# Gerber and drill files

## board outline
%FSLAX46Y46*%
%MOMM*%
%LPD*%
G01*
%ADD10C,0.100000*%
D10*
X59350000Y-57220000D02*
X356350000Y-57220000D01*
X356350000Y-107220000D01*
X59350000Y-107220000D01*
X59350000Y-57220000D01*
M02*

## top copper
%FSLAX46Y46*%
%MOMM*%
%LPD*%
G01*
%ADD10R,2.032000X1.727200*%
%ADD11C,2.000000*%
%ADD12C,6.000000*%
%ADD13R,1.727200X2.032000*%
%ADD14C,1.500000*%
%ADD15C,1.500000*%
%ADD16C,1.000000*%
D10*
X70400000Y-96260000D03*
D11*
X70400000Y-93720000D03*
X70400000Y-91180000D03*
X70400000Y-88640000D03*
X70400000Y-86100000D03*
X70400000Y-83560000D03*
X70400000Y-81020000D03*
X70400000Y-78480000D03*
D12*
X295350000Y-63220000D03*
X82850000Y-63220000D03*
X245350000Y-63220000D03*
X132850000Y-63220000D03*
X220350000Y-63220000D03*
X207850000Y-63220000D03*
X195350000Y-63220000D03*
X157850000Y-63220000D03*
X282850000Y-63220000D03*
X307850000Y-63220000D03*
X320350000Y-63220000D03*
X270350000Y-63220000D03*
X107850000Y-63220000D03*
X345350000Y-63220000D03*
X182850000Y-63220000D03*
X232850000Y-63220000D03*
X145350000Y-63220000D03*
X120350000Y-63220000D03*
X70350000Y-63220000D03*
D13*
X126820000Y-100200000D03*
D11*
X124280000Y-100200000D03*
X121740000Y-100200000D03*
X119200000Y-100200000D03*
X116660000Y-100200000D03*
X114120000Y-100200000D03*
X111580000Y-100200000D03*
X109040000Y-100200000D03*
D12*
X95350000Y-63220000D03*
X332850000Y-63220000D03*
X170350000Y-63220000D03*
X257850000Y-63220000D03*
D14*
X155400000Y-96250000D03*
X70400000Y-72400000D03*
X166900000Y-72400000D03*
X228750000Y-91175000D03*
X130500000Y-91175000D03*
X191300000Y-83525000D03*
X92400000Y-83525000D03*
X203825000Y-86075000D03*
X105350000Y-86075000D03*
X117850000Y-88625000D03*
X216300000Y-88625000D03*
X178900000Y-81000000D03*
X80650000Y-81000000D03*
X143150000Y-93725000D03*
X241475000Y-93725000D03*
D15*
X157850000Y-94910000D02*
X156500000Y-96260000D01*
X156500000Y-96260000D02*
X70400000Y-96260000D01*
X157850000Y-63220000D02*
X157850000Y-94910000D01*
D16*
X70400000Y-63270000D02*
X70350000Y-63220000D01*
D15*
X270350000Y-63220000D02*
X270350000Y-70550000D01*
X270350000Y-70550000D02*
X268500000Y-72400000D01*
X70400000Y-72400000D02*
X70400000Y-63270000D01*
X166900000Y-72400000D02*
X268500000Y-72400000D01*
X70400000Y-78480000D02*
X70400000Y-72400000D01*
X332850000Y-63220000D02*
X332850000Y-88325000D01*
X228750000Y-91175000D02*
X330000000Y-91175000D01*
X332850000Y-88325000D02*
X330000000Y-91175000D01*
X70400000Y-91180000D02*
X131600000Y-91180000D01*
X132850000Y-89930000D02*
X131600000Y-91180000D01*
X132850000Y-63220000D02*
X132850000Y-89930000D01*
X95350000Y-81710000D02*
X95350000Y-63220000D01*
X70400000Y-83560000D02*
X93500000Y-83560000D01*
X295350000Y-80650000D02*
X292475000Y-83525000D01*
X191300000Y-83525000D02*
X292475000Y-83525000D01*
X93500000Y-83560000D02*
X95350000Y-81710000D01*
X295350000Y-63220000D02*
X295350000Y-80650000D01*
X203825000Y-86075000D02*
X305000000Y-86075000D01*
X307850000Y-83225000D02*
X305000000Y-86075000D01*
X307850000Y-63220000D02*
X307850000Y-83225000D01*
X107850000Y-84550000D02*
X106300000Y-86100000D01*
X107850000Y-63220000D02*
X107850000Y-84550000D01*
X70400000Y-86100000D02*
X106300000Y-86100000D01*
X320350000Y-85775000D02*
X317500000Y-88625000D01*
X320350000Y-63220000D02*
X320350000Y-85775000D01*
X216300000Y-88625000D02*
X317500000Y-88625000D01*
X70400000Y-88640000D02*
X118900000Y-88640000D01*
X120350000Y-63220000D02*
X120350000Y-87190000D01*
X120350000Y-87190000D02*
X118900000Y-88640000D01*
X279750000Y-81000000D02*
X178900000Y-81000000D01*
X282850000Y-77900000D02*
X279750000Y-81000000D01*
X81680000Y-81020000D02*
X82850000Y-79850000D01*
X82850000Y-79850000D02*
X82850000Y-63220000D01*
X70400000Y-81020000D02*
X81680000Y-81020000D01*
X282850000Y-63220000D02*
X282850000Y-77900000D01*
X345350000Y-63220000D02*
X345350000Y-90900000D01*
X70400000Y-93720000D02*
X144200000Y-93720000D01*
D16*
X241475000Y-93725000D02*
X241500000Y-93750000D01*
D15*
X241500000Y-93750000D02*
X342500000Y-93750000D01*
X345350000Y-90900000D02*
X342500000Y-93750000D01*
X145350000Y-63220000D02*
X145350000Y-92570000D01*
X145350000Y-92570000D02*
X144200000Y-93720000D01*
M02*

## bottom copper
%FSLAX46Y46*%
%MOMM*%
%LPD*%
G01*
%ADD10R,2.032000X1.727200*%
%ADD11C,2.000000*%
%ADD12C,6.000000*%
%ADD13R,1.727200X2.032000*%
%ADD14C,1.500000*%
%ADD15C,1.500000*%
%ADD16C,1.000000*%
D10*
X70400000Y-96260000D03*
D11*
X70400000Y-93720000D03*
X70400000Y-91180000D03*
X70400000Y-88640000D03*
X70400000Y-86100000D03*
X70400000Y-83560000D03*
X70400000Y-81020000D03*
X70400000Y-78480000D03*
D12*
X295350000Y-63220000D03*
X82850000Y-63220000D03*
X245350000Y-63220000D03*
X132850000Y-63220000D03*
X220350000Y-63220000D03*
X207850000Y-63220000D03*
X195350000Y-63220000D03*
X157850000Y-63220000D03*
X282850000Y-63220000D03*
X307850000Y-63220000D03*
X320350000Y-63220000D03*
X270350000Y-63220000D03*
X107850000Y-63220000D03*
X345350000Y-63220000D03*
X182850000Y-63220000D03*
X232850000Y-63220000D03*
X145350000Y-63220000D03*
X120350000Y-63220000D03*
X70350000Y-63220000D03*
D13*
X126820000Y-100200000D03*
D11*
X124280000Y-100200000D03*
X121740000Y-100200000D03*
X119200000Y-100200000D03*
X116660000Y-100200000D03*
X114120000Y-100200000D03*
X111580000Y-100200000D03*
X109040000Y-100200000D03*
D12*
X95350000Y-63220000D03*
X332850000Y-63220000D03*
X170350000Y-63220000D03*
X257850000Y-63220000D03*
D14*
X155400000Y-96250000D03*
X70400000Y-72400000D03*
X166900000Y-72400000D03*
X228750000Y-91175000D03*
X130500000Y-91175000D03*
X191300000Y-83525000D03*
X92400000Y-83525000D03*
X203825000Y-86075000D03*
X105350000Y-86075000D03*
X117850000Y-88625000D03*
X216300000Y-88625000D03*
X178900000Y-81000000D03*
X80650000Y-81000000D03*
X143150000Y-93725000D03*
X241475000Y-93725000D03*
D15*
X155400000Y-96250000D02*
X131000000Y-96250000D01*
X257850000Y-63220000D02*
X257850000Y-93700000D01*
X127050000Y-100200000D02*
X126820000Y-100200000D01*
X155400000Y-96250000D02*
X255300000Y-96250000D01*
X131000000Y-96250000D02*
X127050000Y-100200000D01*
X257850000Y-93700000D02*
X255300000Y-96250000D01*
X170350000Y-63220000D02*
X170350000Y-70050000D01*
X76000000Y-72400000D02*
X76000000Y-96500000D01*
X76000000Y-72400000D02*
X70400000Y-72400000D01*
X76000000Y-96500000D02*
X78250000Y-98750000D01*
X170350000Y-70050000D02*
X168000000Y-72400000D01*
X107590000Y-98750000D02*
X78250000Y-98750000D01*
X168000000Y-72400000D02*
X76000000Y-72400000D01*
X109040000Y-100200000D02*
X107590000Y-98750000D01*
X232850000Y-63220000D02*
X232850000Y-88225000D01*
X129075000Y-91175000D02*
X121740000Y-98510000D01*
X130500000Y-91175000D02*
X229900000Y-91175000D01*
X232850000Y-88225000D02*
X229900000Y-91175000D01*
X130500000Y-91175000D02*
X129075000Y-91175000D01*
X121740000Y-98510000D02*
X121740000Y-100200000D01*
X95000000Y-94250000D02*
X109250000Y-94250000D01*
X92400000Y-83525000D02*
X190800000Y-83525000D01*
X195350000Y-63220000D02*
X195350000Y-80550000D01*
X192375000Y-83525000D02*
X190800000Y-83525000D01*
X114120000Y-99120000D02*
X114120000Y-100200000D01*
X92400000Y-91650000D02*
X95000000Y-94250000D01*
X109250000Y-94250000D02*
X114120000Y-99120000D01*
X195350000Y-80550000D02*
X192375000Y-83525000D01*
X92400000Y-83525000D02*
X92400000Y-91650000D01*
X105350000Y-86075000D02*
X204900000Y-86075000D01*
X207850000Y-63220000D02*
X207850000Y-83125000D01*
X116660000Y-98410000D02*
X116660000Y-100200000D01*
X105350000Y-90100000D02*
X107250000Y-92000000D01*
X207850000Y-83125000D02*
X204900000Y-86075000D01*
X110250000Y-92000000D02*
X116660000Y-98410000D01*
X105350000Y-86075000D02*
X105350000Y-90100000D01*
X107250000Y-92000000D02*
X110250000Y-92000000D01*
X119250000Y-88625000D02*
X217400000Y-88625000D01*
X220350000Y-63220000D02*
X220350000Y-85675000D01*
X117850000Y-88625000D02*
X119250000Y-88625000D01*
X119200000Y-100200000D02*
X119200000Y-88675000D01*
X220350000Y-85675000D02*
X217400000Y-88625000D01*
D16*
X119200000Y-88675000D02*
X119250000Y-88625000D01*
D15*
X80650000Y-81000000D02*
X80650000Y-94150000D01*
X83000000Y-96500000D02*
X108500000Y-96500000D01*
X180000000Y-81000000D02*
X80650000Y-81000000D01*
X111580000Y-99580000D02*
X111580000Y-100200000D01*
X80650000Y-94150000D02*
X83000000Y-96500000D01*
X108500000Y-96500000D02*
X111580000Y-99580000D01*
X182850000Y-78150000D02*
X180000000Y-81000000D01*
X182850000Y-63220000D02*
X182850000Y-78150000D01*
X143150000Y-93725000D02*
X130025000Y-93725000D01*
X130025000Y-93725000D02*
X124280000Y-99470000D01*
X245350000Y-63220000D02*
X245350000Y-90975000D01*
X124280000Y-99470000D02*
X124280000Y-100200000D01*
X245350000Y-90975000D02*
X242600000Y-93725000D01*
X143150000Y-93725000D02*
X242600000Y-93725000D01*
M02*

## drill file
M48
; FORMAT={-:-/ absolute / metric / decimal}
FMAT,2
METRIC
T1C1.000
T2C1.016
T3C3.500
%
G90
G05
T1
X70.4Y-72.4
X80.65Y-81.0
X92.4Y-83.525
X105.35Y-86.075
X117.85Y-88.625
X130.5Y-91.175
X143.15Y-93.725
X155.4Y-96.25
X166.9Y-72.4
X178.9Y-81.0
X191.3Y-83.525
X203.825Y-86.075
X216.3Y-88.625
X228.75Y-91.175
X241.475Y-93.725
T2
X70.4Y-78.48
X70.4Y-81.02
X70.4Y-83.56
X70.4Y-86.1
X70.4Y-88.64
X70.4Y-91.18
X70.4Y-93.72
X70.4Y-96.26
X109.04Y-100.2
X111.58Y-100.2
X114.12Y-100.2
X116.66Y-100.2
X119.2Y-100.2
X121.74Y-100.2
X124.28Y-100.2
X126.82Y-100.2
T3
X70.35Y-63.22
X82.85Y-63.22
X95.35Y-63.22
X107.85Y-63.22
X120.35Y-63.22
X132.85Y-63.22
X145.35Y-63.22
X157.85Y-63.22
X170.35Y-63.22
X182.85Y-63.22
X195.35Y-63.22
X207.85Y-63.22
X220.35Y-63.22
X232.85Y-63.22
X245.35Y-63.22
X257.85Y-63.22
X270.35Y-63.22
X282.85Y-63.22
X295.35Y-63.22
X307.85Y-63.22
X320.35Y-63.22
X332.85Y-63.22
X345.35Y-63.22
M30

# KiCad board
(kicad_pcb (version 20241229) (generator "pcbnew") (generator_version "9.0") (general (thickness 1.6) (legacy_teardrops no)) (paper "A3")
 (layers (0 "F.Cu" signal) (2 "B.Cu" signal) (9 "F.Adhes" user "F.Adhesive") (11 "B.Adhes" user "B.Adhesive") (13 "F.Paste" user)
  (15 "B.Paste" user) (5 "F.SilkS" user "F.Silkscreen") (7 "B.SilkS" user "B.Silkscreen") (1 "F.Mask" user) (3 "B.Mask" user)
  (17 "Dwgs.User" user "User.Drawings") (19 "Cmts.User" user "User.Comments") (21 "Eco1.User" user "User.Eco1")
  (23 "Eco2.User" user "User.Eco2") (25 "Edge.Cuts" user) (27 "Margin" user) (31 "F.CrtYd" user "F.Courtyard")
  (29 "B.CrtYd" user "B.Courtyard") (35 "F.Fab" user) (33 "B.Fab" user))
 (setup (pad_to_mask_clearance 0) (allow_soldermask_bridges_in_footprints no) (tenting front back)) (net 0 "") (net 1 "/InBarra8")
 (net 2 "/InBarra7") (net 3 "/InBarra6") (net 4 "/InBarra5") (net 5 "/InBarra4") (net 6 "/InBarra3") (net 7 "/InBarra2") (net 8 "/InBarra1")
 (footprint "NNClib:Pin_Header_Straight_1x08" (layer "F.Cu") (at 70.4 96.26 180)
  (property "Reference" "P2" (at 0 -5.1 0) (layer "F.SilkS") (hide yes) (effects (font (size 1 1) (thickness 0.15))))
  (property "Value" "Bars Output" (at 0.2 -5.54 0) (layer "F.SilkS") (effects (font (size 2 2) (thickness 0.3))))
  (pad "1" thru_hole rect (at 0 0 180) (size 2.032 1.7272) (drill 1.016) (layers "*.Cu" "*.Mask" "F.SilkS") (remove_unused_layers no)
   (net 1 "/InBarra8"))
  (pad "2" thru_hole circle (at 0 2.54 180) (size 2 2) (drill 1.016) (layers "*.Cu" "*.Mask" "F.SilkS") (remove_unused_layers no)
   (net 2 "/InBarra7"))
  (pad "3" thru_hole circle (at 0 5.08 180) (size 2 2) (drill 1.016) (layers "*.Cu" "*.Mask" "F.SilkS") (remove_unused_layers no)
   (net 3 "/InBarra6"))
  (pad "4" thru_hole circle (at 0 7.62 180) (size 2 2) (drill 1.016) (layers "*.Cu" "*.Mask" "F.SilkS") (remove_unused_layers no)
   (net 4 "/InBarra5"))
  (pad "5" thru_hole circle (at 0 10.16 180) (size 2 2) (drill 1.016) (layers "*.Cu" "*.Mask" "F.SilkS") (remove_unused_layers no)
   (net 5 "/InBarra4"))
  (pad "6" thru_hole circle (at 0 12.7 180) (size 2 2) (drill 1.016) (layers "*.Cu" "*.Mask" "F.SilkS") (remove_unused_layers no)
   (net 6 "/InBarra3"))
  (pad "7" thru_hole circle (at 0 15.24 180) (size 2 2) (drill 1.016) (layers "*.Cu" "*.Mask" "F.SilkS") (remove_unused_layers no)
   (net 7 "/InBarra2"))
  (pad "8" thru_hole circle (at 0 17.78 180) (size 2 2) (drill 1.016) (layers "*.Cu" "*.Mask" "F.SilkS") (remove_unused_layers no)
   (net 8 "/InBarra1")))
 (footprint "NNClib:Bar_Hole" (layer "F.Cu") (at 295.35 63.22)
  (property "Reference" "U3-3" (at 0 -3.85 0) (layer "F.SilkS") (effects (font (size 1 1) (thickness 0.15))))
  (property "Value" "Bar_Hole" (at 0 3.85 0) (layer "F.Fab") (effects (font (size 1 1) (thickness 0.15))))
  (pad "1" thru_hole circle (at 0 0) (size 6 6) (drill 3.5) (layers "*.Cu" "*.Mask" "F.SilkS") (remove_unused_layers no) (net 6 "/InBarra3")))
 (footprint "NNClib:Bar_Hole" (layer "F.Cu") (at 82.85 63.22)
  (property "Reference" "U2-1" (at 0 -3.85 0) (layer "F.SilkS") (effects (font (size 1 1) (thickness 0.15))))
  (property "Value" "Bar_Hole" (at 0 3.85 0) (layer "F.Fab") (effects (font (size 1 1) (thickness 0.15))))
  (pad "1" thru_hole circle (at 0 0) (size 6 6) (drill 3.5) (layers "*.Cu" "*.Mask" "F.SilkS") (remove_unused_layers no) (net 7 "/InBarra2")))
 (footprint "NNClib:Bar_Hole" (layer "F.Cu") (at 245.35 63.22)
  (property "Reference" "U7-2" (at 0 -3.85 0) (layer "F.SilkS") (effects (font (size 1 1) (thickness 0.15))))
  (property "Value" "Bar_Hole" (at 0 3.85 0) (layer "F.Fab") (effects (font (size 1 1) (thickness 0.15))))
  (pad "1" thru_hole circle (at 0 0) (size 6 6) (drill 3.5) (layers "*.Cu" "*.Mask" "F.SilkS") (remove_unused_layers no) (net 2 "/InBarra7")))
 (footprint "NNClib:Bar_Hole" (layer "F.Cu") (at 132.85 63.22)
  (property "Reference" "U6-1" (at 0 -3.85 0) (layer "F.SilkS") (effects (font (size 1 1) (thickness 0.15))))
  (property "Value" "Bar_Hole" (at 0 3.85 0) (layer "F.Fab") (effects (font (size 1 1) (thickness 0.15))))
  (pad "1" thru_hole circle (at 0 0) (size 6 6) (drill 3.5) (layers "*.Cu" "*.Mask" "F.SilkS") (remove_unused_layers no) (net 3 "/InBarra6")))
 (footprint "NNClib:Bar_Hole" (layer "F.Cu") (at 220.35 63.22)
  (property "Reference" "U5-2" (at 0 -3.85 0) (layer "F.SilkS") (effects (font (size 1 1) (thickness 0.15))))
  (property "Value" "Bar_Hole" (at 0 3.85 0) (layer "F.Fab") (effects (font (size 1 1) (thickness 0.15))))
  (pad "1" thru_hole circle (at 0 0) (size 6 6) (drill 3.5) (layers "*.Cu" "*.Mask" "F.SilkS") (remove_unused_layers no) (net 4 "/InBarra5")))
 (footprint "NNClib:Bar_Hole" (layer "F.Cu") (at 207.85 63.22)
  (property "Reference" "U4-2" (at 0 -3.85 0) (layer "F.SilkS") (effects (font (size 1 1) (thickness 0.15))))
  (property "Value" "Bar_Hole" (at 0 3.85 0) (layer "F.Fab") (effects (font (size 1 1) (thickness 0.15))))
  (pad "1" thru_hole circle (at 0 0) (size 6 6) (drill 3.5) (layers "*.Cu" "*.Mask" "F.SilkS") (remove_unused_layers no) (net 5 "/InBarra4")))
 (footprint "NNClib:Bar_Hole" (layer "F.Cu") (at 195.35 63.22)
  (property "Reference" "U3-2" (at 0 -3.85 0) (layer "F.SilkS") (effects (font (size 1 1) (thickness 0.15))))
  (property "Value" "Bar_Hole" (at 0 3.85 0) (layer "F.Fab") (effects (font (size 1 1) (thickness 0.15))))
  (pad "1" thru_hole circle (at 0 0) (size 6 6) (drill 3.5) (layers "*.Cu" "*.Mask" "F.SilkS") (remove_unused_layers no) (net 6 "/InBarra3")))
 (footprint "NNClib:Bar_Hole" (layer "F.Cu") (at 157.85 63.22)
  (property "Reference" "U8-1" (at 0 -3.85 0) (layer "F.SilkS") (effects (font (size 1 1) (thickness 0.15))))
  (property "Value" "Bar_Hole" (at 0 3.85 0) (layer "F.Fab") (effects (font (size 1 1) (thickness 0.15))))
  (pad "1" thru_hole circle (at 0 0) (size 6 6) (drill 3.5) (layers "*.Cu" "*.Mask" "F.SilkS") (remove_unused_layers no) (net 1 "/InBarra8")))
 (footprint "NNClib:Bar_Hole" (layer "F.Cu") (at 282.85 63.22)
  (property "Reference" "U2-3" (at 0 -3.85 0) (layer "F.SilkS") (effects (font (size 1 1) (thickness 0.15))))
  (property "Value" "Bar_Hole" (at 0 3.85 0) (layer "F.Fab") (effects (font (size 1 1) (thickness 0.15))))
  (pad "1" thru_hole circle (at 0 0) (size 6 6) (drill 3.5) (layers "*.Cu" "*.Mask" "F.SilkS") (remove_unused_layers no) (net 7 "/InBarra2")))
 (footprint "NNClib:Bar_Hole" (layer "F.Cu") (at 307.85 63.22)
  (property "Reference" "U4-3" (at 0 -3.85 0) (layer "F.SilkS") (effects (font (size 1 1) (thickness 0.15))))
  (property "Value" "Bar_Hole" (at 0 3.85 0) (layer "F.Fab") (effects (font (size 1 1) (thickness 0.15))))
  (pad "1" thru_hole circle (at 0 0) (size 6 6) (drill 3.5) (layers "*.Cu" "*.Mask" "F.SilkS") (remove_unused_layers no) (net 5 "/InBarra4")))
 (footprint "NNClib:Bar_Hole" (layer "F.Cu") (at 320.35 63.22)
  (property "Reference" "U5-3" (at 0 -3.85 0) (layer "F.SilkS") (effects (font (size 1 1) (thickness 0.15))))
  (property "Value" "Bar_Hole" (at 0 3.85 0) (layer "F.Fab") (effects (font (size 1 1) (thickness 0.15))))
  (pad "1" thru_hole circle (at 0 0) (size 6 6) (drill 3.5) (layers "*.Cu" "*.Mask" "F.SilkS") (remove_unused_layers no) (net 4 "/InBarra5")))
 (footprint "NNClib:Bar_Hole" (layer "F.Cu") (at 270.35 63.22)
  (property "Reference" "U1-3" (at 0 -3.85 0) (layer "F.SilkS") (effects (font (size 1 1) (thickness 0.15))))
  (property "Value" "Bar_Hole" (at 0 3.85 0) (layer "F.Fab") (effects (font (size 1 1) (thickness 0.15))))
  (pad "1" thru_hole circle (at 0 0) (size 6 6) (drill 3.5) (layers "*.Cu" "*.Mask" "F.SilkS") (remove_unused_layers no) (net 8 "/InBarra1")))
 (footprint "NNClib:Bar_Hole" (layer "F.Cu") (at 107.85 63.22)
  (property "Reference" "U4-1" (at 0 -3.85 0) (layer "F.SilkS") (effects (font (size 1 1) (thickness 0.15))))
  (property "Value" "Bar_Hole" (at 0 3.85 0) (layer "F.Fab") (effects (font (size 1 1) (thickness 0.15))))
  (pad "1" thru_hole circle (at 0 0) (size 6 6) (drill 3.5) (layers "*.Cu" "*.Mask" "F.SilkS") (remove_unused_layers no) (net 5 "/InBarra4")))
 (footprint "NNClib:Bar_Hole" (layer "F.Cu") (at 345.35 63.22)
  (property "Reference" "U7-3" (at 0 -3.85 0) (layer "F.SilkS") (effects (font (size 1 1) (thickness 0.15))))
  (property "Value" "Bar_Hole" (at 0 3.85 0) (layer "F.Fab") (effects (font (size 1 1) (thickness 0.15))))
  (pad "1" thru_hole circle (at 0 0) (size 6 6) (drill 3.5) (layers "*.Cu" "*.Mask" "F.SilkS") (remove_unused_layers no) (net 2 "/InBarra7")))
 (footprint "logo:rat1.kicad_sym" (layer "F.Cu") (at 341.4 89.8)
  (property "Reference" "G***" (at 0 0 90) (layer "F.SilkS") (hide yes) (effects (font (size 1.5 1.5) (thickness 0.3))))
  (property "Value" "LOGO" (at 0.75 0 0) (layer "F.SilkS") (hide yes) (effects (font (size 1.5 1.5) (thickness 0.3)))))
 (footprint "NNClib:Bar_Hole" (layer "F.Cu") (at 182.85 63.22)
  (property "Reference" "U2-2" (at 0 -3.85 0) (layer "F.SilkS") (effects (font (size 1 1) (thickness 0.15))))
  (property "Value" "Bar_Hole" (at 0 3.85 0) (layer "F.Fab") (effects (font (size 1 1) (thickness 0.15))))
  (pad "1" thru_hole circle (at 0 0) (size 6 6) (drill 3.5) (layers "*.Cu" "*.Mask" "F.SilkS") (remove_unused_layers no) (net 7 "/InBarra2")))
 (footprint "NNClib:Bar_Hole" (layer "F.Cu") (at 232.85 63.22)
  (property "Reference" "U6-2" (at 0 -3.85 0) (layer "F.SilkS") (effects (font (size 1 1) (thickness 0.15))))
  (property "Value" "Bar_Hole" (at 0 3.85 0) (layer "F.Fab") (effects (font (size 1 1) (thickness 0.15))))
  (pad "1" thru_hole circle (at 0 0) (size 6 6) (drill 3.5) (layers "*.Cu" "*.Mask" "F.SilkS") (remove_unused_layers no) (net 3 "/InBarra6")))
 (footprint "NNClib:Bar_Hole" (layer "F.Cu") (at 145.35 63.22)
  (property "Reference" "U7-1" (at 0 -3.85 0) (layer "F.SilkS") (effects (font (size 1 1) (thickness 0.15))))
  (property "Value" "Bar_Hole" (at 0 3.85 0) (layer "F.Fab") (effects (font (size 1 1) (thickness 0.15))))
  (pad "1" thru_hole circle (at 0 0) (size 6 6) (drill 3.5) (layers "*.Cu" "*.Mask" "F.SilkS") (remove_unused_layers no) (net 2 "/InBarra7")))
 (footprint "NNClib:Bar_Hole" (layer "F.Cu") (at 120.35 63.22)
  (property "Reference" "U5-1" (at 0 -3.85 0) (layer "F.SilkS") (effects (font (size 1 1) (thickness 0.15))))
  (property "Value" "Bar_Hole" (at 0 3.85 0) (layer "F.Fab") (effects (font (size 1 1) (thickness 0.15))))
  (pad "1" thru_hole circle (at 0 0) (size 6 6) (drill 3.5) (layers "*.Cu" "*.Mask" "F.SilkS") (remove_unused_layers no) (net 4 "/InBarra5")))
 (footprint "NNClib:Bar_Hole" (layer "F.Cu") (at 70.35 63.22)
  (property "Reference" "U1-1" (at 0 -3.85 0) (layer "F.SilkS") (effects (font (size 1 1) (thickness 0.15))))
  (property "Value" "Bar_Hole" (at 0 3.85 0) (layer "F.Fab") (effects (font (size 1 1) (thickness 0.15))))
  (pad "1" thru_hole circle (at 0 0) (size 6 6) (drill 3.5) (layers "*.Cu" "*.Mask" "F.SilkS") (remove_unused_layers no) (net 8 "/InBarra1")))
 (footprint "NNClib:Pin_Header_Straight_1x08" (layer "F.Cu") (at 126.82 100.2 -90)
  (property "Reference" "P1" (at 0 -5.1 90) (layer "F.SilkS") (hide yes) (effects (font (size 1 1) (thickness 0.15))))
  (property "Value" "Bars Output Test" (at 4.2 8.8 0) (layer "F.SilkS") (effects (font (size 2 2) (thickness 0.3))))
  (pad "1" thru_hole rect (at 0 0 270) (size 2.032 1.7272) (drill 1.016) (layers "*.Cu" "*.Mask" "F.SilkS") (remove_unused_layers no)
   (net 1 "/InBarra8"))
  (pad "2" thru_hole circle (at 0 2.54 270) (size 2 2) (drill 1.016) (layers "*.Cu" "*.Mask" "F.SilkS") (remove_unused_layers no)
   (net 2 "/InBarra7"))
  (pad "3" thru_hole circle (at 0 5.08 270) (size 2 2) (drill 1.016) (layers "*.Cu" "*.Mask" "F.SilkS") (remove_unused_layers no)
   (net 3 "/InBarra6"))
  (pad "4" thru_hole circle (at 0 7.62 270) (size 2 2) (drill 1.016) (layers "*.Cu" "*.Mask" "F.SilkS") (remove_unused_layers no)
   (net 4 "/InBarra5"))
  (pad "5" thru_hole circle (at 0 10.16 270) (size 2 2) (drill 1.016) (layers "*.Cu" "*.Mask" "F.SilkS") (remove_unused_layers no)
   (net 5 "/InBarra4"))
  (pad "6" thru_hole circle (at 0 12.7 270) (size 2 2) (drill 1.016) (layers "*.Cu" "*.Mask" "F.SilkS") (remove_unused_layers no)
   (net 6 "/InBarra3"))
  (pad "7" thru_hole circle (at 0 15.24 270) (size 2 2) (drill 1.016) (layers "*.Cu" "*.Mask" "F.SilkS") (remove_unused_layers no)
   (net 7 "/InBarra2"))
  (pad "8" thru_hole circle (at 0 17.78 270) (size 2 2) (drill 1.016) (layers "*.Cu" "*.Mask" "F.SilkS") (remove_unused_layers no)
   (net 8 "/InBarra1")))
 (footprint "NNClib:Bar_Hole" (layer "F.Cu") (at 95.35 63.22)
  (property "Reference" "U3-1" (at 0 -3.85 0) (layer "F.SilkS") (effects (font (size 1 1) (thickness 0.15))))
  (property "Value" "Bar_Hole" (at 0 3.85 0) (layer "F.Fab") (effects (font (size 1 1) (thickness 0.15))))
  (pad "1" thru_hole circle (at 0 0) (size 6 6) (drill 3.5) (layers "*.Cu" "*.Mask" "F.SilkS") (remove_unused_layers no) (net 6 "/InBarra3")))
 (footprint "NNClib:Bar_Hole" (layer "F.Cu") (at 332.85 63.22)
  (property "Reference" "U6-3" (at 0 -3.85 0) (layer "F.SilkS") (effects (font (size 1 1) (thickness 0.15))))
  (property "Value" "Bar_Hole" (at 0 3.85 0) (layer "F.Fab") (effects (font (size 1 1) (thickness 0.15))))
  (pad "1" thru_hole circle (at 0 0) (size 6 6) (drill 3.5) (layers "*.Cu" "*.Mask" "F.SilkS") (remove_unused_layers no) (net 3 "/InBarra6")))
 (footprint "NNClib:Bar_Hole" (layer "F.Cu") (at 170.35 63.22)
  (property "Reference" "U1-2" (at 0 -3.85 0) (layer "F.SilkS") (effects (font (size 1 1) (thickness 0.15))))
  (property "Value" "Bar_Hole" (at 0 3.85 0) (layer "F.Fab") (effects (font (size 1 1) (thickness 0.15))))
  (pad "1" thru_hole circle (at 0 0) (size 6 6) (drill 3.5) (layers "*.Cu" "*.Mask" "F.SilkS") (remove_unused_layers no) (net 8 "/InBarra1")))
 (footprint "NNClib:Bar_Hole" (layer "F.Cu") (at 257.85 63.22)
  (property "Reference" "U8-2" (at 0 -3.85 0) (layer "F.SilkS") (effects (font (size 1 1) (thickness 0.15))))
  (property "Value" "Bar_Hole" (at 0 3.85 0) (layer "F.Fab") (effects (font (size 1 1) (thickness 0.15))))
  (pad "1" thru_hole circle (at 0 0) (size 6 6) (drill 3.5) (layers "*.Cu" "*.Mask" "F.SilkS") (remove_unused_layers no) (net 1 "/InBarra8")))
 (gr_rect (start 59.35 57.22) (end 356.35 107.22) (stroke (width 0.1) (type solid)) (fill no) (layer "Edge.Cuts"))
 (segment (start 157.85 94.91) (end 156.5 96.26) (width 1.5) (layer "F.Cu") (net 1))
 (segment (start 156.5 96.26) (end 70.4 96.26) (width 1.5) (layer "F.Cu") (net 1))
 (segment (start 157.85 63.22) (end 157.85 94.91) (width 1.5) (layer "F.Cu") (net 1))
 (via (at 155.4 96.25) (size 1.5) (drill 1) (layers "F.Cu" "B.Cu") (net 1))
 (segment (start 155.4 96.25) (end 131 96.25) (width 1.5) (layer "B.Cu") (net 1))
 (segment (start 257.85 63.22) (end 257.85 93.7) (width 1.5) (layer "B.Cu") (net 1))
 (segment (start 127.05 100.2) (end 126.82 100.2) (width 1.5) (layer "B.Cu") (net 1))
 (segment (start 155.4 96.25) (end 255.3 96.25) (width 1.5) (layer "B.Cu") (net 1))
 (segment (start 131 96.25) (end 127.05 100.2) (width 1.5) (layer "B.Cu") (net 1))
 (segment (start 257.85 93.7) (end 255.3 96.25) (width 1.5) (layer "B.Cu") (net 1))
 (segment (start 70.4 63.27) (end 70.35 63.22) (width 1) (layer "F.Cu") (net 8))
 (segment (start 270.35 63.22) (end 270.35 70.55) (width 1.5) (layer "F.Cu") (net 8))
 (segment (start 270.35 70.55) (end 268.5 72.4) (width 1.5) (layer "F.Cu") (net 8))
 (segment (start 70.4 72.4) (end 70.4 63.27) (width 1.5) (layer "F.Cu") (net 8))
 (segment (start 166.9 72.4) (end 268.5 72.4) (width 1.5) (layer "F.Cu") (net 8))
 (segment (start 70.4 78.48) (end 70.4 72.4) (width 1.5) (layer "F.Cu") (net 8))
 (via (at 70.4 72.4) (size 1.5) (drill 1) (layers "F.Cu" "B.Cu") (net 8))
 (via (at 166.9 72.4) (size 1.5) (drill 1) (layers "F.Cu" "B.Cu") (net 8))
 (segment (start 170.35 63.22) (end 170.35 70.05) (width 1.5) (layer "B.Cu") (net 8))
 (segment (start 76 72.4) (end 76 96.5) (width 1.5) (layer "B.Cu") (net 8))
 (segment (start 76 72.4) (end 70.4 72.4) (width 1.5) (layer "B.Cu") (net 8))
 (segment (start 76 96.5) (end 78.25 98.75) (width 1.5) (layer "B.Cu") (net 8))
 (segment (start 170.35 70.05) (end 168 72.4) (width 1.5) (layer "B.Cu") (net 8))
 (segment (start 107.59 98.75) (end 78.25 98.75) (width 1.5) (layer "B.Cu") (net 8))
 (segment (start 168 72.4) (end 76 72.4) (width 1.5) (layer "B.Cu") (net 8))
 (segment (start 109.04 100.2) (end 107.59 98.75) (width 1.5) (layer "B.Cu") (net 8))
 (segment (start 332.85 63.22) (end 332.85 88.325) (width 1.5) (layer "F.Cu") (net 3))
 (segment (start 228.75 91.175) (end 330 91.175) (width 1.5) (layer "F.Cu") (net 3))
 (segment (start 332.85 88.325) (end 330 91.175) (width 1.5) (layer "F.Cu") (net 3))
 (segment (start 70.4 91.18) (end 131.6 91.18) (width 1.5) (layer "F.Cu") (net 3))
 (segment (start 132.85 89.93) (end 131.6 91.18) (width 1.5) (layer "F.Cu") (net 3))
 (segment (start 132.85 63.22) (end 132.85 89.93) (width 1.5) (layer "F.Cu") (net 3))
 (via (at 228.75 91.175) (size 1.5) (drill 1) (layers "F.Cu" "B.Cu") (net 3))
 (via (at 130.5 91.175) (size 1.5) (drill 1) (layers "F.Cu" "B.Cu") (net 3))
 (segment (start 232.85 63.22) (end 232.85 88.225) (width 1.5) (layer "B.Cu") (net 3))
 (segment (start 129.075 91.175) (end 121.74 98.51) (width 1.5) (layer "B.Cu") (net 3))
 (segment (start 130.5 91.175) (end 229.9 91.175) (width 1.5) (layer "B.Cu") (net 3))
 (segment (start 232.85 88.225) (end 229.9 91.175) (width 1.5) (layer "B.Cu") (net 3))
 (segment (start 130.5 91.175) (end 129.075 91.175) (width 1.5) (layer "B.Cu") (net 3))
 (segment (start 121.74 98.51) (end 121.74 100.2) (width 1.5) (layer "B.Cu") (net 3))
 (segment (start 95.35 81.71) (end 95.35 63.22) (width 1.5) (layer "F.Cu") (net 6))
 (segment (start 70.4 83.56) (end 93.5 83.56) (width 1.5) (layer "F.Cu") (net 6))
 (segment (start 295.35 80.65) (end 292.475 83.525) (width 1.5) (layer "F.Cu") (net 6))
 (segment (start 191.3 83.525) (end 292.475 83.525) (width 1.5) (layer "F.Cu") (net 6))
 (segment (start 93.5 83.56) (end 95.35 81.71) (width 1.5) (layer "F.Cu") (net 6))
 (segment (start 295.35 63.22) (end 295.35 80.65) (width 1.5) (layer "F.Cu") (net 6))
 (via (at 191.3 83.525) (size 1.5) (drill 1) (layers "F.Cu" "B.Cu") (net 6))
 (via (at 92.4 83.525) (size 1.5) (drill 1) (layers "F.Cu" "B.Cu") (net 6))
 (segment (start 95 94.25) (end 109.25 94.25) (width 1.5) (layer "B.Cu") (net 6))
 (segment (start 92.4 83.525) (end 190.8 83.525) (width 1.5) (layer "B.Cu") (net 6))
 (segment (start 195.35 63.22) (end 195.35 80.55) (width 1.5) (layer "B.Cu") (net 6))
 (segment (start 192.375 83.525) (end 190.8 83.525) (width 1.5) (layer "B.Cu") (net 6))
 (segment (start 114.12 99.12) (end 114.12 100.2) (width 1.5) (layer "B.Cu") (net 6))
 (segment (start 92.4 91.65) (end 95 94.25) (width 1.5) (layer "B.Cu") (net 6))
 (segment (start 109.25 94.25) (end 114.12 99.12) (width 1.5) (layer "B.Cu") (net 6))
 (segment (start 195.35 80.55) (end 192.375 83.525) (width 1.5) (layer "B.Cu") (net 6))
 (segment (start 92.4 83.525) (end 92.4 91.65) (width 1.5) (layer "B.Cu") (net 6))
 (segment (start 203.825 86.075) (end 305 86.075) (width 1.5) (layer "F.Cu") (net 5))
 (segment (start 307.85 83.225) (end 305 86.075) (width 1.5) (layer "F.Cu") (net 5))
 (segment (start 307.85 63.22) (end 307.85 83.225) (width 1.5) (layer "F.Cu") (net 5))
 (segment (start 107.85 84.55) (end 106.3 86.1) (width 1.5) (layer "F.Cu") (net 5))
 (segment (start 107.85 63.22) (end 107.85 84.55) (width 1.5) (layer "F.Cu") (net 5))
 (segment (start 70.4 86.1) (end 106.3 86.1) (width 1.5) (layer "F.Cu") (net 5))
 (via (at 203.825 86.075) (size 1.5) (drill 1) (layers "F.Cu" "B.Cu") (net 5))
 (via (at 105.35 86.075) (size 1.5) (drill 1) (layers "F.Cu" "B.Cu") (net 5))
 (segment (start 105.35 86.075) (end 204.9 86.075) (width 1.5) (layer "B.Cu") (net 5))
 (segment (start 207.85 63.22) (end 207.85 83.125) (width 1.5) (layer "B.Cu") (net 5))
 (segment (start 116.66 98.41) (end 116.66 100.2) (width 1.5) (layer "B.Cu") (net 5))
 (segment (start 105.35 90.1) (end 107.25 92) (width 1.5) (layer "B.Cu") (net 5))
 (segment (start 207.85 83.125) (end 204.9 86.075) (width 1.5) (layer "B.Cu") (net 5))
 (segment (start 110.25 92) (end 116.66 98.41) (width 1.5) (layer "B.Cu") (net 5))
 (segment (start 105.35 86.075) (end 105.35 90.1) (width 1.5) (layer "B.Cu") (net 5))
 (segment (start 107.25 92) (end 110.25 92) (width 1.5) (layer "B.Cu") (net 5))
 (segment (start 320.35 85.775) (end 317.5 88.625) (width 1.5) (layer "F.Cu") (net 4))
 (segment (start 320.35 63.22) (end 320.35 85.775) (width 1.5) (layer "F.Cu") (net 4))
 (segment (start 216.3 88.625) (end 317.5 88.625) (width 1.5) (layer "F.Cu") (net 4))
 (segment (start 70.4 88.64) (end 118.9 88.64) (width 1.5) (layer "F.Cu") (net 4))
 (segment (start 120.35 63.22) (end 120.35 87.19) (width 1.5) (layer "F.Cu") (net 4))
 (segment (start 120.35 87.19) (end 118.9 88.64) (width 1.5) (layer "F.Cu") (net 4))
 (via (at 117.85 88.625) (size 1.5) (drill 1) (layers "F.Cu" "B.Cu") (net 4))
 (via (at 216.3 88.625) (size 1.5) (drill 1) (layers "F.Cu" "B.Cu") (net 4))
 (segment (start 119.25 88.625) (end 217.4 88.625) (width 1.5) (layer "B.Cu") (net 4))
 (segment (start 220.35 63.22) (end 220.35 85.675) (width 1.5) (layer "B.Cu") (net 4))
 (segment (start 117.85 88.625) (end 119.25 88.625) (width 1.5) (layer "B.Cu") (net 4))
 (segment (start 119.2 100.2) (end 119.2 88.675) (width 1.5) (layer "B.Cu") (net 4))
 (segment (start 220.35 85.675) (end 217.4 88.625) (width 1.5) (layer "B.Cu") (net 4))
 (segment (start 119.2 88.675) (end 119.25 88.625) (width 1) (layer "B.Cu") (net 4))
 (segment (start 279.75 81) (end 178.9 81) (width 1.5) (layer "F.Cu") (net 7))
 (segment (start 282.85 77.9) (end 279.75 81) (width 1.5) (layer "F.Cu") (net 7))
 (segment (start 81.68 81.02) (end 82.85 79.85) (width 1.5) (layer "F.Cu") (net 7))
 (segment (start 82.85 79.85) (end 82.85 63.22) (width 1.5) (layer "F.Cu") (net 7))
 (segment (start 70.4 81.02) (end 81.68 81.02) (width 1.5) (layer "F.Cu") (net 7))
 (segment (start 282.85 63.22) (end 282.85 77.9) (width 1.5) (layer "F.Cu") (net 7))
 (via (at 178.9 81) (size 1.5) (drill 1) (layers "F.Cu" "B.Cu") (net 7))
 (via (at 80.65 81) (size 1.5) (drill 1) (layers "F.Cu" "B.Cu") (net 7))
 (segment (start 80.65 81) (end 80.65 94.15) (width 1.5) (layer "B.Cu") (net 7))
 (segment (start 83 96.5) (end 108.5 96.5) (width 1.5) (layer "B.Cu") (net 7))
 (segment (start 180 81) (end 80.65 81) (width 1.5) (layer "B.Cu") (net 7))
 (segment (start 111.58 99.58) (end 111.58 100.2) (width 1.5) (layer "B.Cu") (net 7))
 (segment (start 80.65 94.15) (end 83 96.5) (width 1.5) (layer "B.Cu") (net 7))
 (segment (start 108.5 96.5) (end 111.58 99.58) (width 1.5) (layer "B.Cu") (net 7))
 (segment (start 182.85 78.15) (end 180 81) (width 1.5) (layer "B.Cu") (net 7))
 (segment (start 182.85 63.22) (end 182.85 78.15) (width 1.5) (layer "B.Cu") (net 7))
 (segment (start 345.35 63.22) (end 345.35 90.9) (width 1.5) (layer "F.Cu") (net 2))
 (segment (start 70.4 93.72) (end 144.2 93.72) (width 1.5) (layer "F.Cu") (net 2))
 (segment (start 241.475 93.725) (end 241.5 93.75) (width 1) (layer "F.Cu") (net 2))
 (segment (start 241.5 93.75) (end 342.5 93.75) (width 1.5) (layer "F.Cu") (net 2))
 (segment (start 345.35 90.9) (end 342.5 93.75) (width 1.5) (layer "F.Cu") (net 2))
 (segment (start 145.35 63.22) (end 145.35 92.57) (width 1.5) (layer "F.Cu") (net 2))
 (segment (start 145.35 92.57) (end 144.2 93.72) (width 1.5) (layer "F.Cu") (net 2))
 (via (at 143.15 93.725) (size 1.5) (drill 1) (layers "F.Cu" "B.Cu") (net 2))
 (via (at 241.475 93.725) (size 1.5) (drill 1) (layers "F.Cu" "B.Cu") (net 2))
 (segment (start 143.15 93.725) (end 130.025 93.725) (width 1.5) (layer "B.Cu") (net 2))
 (segment (start 130.025 93.725) (end 124.28 99.47) (width 1.5) (layer "B.Cu") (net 2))
 (segment (start 245.35 63.22) (end 245.35 90.975) (width 1.5) (layer "B.Cu") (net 2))
 (segment (start 124.28 99.47) (end 124.28 100.2) (width 1.5) (layer "B.Cu") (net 2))
 (segment (start 245.35 90.975) (end 242.6 93.725) (width 1.5) (layer "B.Cu") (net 2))
 (segment (start 143.15 93.725) (end 242.6 93.725) (width 1.5) (layer "B.Cu") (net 2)))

